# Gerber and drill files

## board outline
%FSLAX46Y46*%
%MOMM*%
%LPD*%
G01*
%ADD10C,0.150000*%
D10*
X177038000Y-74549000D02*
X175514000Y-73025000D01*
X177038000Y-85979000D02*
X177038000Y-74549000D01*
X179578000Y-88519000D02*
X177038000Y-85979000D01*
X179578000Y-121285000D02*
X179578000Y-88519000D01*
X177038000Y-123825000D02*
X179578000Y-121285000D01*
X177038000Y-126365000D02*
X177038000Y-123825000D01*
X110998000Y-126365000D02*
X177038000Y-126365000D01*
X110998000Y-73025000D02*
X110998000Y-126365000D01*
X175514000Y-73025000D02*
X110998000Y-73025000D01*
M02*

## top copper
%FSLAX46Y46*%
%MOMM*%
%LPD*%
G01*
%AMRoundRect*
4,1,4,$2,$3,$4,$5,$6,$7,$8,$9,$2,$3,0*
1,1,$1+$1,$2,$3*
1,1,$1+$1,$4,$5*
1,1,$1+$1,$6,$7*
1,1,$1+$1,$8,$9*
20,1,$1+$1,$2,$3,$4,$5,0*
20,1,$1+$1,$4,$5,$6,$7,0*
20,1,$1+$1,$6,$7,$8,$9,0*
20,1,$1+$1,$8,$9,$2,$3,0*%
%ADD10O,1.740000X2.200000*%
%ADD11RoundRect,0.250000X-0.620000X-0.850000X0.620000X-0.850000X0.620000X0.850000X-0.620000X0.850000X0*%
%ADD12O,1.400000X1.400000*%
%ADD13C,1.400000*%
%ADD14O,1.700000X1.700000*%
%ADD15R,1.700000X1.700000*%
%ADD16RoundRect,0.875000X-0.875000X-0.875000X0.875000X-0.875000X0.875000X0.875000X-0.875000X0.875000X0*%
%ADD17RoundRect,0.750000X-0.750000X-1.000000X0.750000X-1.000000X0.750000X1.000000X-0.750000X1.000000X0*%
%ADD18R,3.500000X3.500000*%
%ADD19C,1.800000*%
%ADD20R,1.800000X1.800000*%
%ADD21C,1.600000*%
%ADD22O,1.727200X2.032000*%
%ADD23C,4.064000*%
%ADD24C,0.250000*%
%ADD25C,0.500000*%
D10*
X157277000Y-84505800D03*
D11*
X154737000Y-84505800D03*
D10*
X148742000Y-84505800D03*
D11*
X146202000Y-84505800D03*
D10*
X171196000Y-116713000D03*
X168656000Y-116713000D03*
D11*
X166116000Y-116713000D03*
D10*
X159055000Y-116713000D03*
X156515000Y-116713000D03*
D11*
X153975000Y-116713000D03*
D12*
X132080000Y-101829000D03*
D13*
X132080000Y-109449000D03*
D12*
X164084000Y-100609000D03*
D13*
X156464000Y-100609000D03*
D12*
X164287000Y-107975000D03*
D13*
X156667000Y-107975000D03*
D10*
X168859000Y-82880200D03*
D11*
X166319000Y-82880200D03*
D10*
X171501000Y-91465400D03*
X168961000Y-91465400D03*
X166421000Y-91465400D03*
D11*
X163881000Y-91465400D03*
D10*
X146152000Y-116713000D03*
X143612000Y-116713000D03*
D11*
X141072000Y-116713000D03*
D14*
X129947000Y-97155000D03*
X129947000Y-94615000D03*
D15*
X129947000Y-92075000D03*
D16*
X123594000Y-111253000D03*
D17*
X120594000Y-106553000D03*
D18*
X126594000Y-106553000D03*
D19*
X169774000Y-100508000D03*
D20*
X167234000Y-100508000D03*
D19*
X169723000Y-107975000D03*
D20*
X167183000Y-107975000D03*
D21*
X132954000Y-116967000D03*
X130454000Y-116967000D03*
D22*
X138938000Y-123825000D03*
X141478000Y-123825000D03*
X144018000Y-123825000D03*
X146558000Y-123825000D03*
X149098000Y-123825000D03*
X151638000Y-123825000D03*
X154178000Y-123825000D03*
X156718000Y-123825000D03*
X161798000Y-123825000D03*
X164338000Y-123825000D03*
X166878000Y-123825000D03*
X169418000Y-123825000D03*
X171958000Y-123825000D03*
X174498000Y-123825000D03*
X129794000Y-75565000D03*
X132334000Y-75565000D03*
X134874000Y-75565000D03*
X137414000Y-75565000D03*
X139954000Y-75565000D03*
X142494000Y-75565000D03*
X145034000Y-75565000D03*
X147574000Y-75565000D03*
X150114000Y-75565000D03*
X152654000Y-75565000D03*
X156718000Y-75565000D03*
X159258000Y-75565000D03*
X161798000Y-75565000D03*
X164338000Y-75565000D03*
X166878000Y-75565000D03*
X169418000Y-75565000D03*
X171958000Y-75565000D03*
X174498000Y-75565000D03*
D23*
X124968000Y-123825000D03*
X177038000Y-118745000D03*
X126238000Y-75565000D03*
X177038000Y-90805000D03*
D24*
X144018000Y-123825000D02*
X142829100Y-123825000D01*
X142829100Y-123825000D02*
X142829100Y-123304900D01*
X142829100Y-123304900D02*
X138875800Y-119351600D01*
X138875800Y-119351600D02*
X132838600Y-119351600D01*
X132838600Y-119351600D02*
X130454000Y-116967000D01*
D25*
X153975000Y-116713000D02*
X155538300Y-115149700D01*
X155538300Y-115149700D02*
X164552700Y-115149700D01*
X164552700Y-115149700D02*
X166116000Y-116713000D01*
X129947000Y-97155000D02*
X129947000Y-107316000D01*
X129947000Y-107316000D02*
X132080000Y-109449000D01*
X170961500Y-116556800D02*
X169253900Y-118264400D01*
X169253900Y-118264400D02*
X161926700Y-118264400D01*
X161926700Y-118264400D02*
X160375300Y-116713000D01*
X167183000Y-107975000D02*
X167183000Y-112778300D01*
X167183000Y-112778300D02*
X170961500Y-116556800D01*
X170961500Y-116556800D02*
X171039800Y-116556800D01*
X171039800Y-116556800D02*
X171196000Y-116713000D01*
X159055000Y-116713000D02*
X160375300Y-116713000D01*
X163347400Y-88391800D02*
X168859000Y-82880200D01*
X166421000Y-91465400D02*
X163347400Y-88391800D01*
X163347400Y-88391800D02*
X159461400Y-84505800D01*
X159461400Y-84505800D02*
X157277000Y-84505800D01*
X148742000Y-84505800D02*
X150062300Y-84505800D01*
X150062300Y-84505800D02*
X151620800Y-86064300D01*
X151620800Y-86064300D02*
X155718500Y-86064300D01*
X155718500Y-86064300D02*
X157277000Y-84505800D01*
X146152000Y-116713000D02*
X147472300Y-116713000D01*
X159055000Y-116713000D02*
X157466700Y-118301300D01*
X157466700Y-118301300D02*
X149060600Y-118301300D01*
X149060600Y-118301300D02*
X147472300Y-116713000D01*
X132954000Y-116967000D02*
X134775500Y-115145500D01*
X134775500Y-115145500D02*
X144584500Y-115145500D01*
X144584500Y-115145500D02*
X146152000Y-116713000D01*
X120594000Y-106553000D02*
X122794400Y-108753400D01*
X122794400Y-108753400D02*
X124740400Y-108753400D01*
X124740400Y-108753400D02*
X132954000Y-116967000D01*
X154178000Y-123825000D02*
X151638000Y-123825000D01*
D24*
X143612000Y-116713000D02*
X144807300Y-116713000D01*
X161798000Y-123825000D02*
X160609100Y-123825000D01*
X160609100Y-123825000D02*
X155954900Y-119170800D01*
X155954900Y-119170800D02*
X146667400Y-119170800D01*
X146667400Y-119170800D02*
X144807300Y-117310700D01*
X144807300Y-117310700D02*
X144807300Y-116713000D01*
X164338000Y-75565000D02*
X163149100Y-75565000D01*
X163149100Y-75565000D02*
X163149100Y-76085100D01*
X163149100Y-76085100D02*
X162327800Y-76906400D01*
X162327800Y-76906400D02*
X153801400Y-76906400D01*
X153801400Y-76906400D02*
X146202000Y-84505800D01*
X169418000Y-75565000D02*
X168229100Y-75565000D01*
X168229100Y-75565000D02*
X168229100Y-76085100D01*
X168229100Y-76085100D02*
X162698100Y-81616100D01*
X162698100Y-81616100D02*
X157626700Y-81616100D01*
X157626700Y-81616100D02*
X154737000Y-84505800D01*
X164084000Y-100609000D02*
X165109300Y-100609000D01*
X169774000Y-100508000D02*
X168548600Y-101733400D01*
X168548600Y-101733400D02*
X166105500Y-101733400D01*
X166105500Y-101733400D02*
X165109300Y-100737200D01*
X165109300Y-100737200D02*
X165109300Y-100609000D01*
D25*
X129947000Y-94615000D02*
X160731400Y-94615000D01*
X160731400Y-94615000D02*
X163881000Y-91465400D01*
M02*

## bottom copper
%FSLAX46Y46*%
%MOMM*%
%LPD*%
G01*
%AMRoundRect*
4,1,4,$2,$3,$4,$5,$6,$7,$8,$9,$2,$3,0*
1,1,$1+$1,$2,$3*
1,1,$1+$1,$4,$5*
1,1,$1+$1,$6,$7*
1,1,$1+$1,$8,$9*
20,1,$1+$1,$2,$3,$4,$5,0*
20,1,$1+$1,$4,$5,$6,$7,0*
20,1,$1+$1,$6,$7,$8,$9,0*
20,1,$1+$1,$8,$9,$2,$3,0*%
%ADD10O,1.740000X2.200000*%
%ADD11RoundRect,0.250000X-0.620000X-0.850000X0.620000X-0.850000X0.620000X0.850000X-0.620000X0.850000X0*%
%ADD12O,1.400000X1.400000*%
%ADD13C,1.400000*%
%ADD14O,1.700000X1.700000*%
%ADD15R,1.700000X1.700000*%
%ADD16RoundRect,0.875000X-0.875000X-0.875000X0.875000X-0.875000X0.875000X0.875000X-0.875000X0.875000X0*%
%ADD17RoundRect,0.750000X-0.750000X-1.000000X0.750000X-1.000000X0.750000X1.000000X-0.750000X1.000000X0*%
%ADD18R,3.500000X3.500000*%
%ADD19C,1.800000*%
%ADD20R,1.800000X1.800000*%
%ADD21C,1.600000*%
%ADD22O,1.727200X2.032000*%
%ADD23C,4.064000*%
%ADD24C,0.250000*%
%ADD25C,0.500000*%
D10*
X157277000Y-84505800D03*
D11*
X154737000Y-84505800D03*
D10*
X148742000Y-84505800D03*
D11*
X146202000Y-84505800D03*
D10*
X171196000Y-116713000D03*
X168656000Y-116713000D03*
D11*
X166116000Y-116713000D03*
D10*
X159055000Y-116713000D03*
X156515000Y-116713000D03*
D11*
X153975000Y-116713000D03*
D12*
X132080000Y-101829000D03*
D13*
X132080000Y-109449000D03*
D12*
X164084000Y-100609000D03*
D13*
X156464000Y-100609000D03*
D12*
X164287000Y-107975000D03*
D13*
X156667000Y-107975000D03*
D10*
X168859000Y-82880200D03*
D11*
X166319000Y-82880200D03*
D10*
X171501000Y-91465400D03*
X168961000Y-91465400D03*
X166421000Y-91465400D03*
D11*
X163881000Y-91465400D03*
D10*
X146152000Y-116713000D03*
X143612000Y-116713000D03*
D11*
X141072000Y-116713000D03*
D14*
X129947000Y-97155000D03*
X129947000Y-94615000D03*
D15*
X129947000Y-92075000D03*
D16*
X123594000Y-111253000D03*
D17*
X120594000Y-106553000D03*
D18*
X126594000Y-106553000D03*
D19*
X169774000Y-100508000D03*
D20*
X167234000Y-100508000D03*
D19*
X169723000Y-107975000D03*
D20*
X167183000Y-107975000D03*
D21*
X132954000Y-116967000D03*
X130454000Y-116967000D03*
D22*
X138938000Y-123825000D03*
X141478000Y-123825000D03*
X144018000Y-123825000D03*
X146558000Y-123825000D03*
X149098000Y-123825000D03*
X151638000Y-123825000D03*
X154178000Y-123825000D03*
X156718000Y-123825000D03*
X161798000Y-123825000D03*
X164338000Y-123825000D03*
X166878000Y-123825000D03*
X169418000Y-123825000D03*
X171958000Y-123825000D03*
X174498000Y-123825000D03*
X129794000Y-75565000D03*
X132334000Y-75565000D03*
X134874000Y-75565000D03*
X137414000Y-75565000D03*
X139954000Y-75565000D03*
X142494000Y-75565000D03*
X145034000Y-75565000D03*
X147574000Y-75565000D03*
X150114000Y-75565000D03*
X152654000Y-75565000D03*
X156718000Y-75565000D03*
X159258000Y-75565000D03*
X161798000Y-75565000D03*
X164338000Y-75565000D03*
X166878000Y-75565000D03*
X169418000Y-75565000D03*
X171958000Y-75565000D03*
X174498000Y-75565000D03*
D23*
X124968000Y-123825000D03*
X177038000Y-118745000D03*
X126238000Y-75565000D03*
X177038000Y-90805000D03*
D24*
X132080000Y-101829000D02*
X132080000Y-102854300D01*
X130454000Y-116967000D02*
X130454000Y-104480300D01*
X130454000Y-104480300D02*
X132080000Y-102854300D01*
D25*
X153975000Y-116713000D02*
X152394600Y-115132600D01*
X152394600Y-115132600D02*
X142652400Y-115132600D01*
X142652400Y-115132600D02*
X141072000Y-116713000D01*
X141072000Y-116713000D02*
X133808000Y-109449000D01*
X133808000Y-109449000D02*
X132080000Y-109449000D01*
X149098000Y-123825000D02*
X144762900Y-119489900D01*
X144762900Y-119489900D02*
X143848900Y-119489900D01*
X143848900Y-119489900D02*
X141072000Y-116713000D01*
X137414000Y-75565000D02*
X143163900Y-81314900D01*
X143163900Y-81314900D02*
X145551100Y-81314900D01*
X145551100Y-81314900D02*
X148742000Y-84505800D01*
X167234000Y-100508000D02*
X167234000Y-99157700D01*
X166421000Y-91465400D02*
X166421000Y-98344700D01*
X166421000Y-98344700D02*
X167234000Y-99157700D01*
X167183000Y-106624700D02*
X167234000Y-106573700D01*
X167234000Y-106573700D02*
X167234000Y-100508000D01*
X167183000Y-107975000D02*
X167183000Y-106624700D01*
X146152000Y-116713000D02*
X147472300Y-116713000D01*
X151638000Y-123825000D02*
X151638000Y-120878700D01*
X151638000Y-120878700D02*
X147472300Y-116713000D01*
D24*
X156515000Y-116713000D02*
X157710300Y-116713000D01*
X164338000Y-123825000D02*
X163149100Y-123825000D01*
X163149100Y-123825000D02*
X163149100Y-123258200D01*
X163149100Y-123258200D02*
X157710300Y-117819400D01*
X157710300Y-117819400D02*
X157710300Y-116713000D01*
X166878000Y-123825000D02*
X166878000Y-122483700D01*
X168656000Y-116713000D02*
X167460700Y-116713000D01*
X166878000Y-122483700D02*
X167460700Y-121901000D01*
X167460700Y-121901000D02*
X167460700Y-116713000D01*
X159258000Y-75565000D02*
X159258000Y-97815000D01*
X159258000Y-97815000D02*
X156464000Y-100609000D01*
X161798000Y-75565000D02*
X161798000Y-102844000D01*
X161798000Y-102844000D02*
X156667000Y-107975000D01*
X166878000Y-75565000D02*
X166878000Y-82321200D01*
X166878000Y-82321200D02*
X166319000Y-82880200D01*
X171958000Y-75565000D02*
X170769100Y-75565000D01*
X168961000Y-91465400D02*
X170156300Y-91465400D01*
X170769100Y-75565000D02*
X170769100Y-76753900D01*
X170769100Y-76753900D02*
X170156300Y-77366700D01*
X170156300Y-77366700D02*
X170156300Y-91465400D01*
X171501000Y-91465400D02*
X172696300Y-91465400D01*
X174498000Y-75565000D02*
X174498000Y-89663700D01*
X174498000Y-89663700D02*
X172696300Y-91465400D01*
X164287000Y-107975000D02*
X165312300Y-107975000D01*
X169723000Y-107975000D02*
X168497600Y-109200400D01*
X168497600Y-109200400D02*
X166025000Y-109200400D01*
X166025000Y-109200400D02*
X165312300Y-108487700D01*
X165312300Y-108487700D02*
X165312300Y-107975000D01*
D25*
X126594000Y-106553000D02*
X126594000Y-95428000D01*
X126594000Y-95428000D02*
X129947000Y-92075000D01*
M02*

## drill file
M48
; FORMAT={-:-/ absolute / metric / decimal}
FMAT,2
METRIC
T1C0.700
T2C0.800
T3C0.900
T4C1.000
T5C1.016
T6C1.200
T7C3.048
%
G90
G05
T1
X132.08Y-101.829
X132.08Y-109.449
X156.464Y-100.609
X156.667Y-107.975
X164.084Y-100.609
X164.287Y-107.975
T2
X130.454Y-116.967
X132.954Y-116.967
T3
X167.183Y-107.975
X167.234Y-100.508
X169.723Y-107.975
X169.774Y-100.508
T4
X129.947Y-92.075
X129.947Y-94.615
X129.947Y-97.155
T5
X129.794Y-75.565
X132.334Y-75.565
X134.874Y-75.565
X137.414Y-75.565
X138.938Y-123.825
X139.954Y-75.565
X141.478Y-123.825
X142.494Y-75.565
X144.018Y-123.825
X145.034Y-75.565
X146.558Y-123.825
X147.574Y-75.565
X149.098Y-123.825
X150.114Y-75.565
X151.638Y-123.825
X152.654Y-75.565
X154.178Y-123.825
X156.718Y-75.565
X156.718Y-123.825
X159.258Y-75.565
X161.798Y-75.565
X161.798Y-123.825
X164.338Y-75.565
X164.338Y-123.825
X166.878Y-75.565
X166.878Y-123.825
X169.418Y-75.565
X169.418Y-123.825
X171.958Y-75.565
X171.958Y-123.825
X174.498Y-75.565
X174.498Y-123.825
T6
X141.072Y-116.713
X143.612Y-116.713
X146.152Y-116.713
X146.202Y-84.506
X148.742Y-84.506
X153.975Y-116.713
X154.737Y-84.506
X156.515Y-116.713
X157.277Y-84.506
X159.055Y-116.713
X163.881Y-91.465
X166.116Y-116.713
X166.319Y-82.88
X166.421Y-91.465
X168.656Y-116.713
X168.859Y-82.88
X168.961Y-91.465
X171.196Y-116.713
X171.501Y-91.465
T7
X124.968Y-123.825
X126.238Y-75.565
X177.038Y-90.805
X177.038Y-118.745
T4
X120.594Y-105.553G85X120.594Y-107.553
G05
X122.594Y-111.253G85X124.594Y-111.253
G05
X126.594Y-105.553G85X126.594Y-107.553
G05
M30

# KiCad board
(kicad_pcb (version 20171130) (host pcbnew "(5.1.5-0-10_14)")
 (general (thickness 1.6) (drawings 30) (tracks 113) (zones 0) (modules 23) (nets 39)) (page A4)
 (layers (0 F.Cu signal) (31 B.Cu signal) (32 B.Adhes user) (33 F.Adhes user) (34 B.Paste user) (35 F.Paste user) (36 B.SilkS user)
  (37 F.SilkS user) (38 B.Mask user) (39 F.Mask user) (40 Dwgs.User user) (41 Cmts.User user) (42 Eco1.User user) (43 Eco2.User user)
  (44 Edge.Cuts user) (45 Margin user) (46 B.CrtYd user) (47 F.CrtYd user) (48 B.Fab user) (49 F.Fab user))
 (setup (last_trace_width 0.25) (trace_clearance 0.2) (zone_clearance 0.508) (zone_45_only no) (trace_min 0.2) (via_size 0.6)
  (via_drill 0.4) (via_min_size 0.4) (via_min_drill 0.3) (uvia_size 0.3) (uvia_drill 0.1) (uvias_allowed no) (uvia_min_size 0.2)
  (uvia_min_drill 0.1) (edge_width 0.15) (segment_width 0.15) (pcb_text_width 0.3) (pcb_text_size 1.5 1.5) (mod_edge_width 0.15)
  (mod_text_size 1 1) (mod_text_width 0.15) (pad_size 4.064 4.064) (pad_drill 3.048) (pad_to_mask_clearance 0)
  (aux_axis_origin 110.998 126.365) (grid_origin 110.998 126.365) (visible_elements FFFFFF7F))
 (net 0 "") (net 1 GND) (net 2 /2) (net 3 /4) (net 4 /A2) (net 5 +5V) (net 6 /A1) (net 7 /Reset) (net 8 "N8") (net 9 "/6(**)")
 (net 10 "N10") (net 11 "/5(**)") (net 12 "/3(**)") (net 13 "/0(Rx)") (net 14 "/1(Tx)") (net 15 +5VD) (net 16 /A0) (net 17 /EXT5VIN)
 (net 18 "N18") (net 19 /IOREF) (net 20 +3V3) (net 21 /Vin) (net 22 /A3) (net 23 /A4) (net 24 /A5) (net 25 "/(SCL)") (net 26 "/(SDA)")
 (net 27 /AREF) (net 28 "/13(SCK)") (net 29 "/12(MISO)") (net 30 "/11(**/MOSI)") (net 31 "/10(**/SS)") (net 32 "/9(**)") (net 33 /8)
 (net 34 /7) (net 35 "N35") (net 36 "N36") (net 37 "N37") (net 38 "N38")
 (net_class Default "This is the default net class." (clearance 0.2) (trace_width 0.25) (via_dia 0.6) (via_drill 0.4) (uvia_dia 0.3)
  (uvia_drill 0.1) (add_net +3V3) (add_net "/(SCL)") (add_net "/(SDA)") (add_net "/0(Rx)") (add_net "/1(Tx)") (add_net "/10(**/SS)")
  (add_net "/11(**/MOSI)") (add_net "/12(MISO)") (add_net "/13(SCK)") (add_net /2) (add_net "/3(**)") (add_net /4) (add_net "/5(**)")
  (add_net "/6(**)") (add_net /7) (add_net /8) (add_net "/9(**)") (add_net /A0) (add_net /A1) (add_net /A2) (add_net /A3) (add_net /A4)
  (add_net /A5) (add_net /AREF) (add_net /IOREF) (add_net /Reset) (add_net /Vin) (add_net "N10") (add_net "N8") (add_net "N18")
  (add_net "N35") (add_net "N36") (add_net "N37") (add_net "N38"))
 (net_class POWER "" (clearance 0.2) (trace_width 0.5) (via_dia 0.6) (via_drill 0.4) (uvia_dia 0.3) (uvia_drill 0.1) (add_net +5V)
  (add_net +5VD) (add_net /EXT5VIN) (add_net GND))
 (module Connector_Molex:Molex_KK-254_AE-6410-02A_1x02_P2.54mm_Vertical (layer F.Cu) (at 154.737 84.5058)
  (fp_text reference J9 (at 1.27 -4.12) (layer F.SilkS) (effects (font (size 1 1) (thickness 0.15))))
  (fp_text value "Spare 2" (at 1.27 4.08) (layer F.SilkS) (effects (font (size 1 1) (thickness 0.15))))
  (pad 2 thru_hole oval (at 2.54 0) (size 1.74 2.2) (drill 1.2) (layers *.Cu *.Mask) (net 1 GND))
  (pad 1 thru_hole roundrect (at 0 0) (size 1.74 2.2) (drill 1.2) (layers *.Cu *.Mask) (roundrect_rratio 0.143678) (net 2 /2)))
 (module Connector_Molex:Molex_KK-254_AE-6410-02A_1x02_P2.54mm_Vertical (layer F.Cu) (at 146.202 84.5058)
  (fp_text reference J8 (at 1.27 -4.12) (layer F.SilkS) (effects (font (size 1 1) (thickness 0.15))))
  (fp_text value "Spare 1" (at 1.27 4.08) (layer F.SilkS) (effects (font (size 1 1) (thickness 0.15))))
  (pad 2 thru_hole oval (at 2.54 0) (size 1.74 2.2) (drill 1.2) (layers *.Cu *.Mask) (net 1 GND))
  (pad 1 thru_hole roundrect (at 0 0) (size 1.74 2.2) (drill 1.2) (layers *.Cu *.Mask) (roundrect_rratio 0.143678) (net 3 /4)))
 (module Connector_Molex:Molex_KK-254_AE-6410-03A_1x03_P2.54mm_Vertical (layer F.Cu) (at 166.116 116.713)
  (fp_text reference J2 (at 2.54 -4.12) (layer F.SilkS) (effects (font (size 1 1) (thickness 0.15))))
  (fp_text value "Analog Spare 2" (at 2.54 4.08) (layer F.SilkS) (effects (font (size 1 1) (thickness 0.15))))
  (pad 3 thru_hole oval (at 5.08 0) (size 1.74 2.2) (drill 1.2) (layers *.Cu *.Mask) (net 1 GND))
  (pad 2 thru_hole oval (at 2.54 0) (size 1.74 2.2) (drill 1.2) (layers *.Cu *.Mask) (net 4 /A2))
  (pad 1 thru_hole roundrect (at 0 0) (size 1.74 2.2) (drill 1.2) (layers *.Cu *.Mask) (roundrect_rratio 0.143678) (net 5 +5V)))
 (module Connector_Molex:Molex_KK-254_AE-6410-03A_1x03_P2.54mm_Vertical (layer F.Cu) (at 153.975 116.713)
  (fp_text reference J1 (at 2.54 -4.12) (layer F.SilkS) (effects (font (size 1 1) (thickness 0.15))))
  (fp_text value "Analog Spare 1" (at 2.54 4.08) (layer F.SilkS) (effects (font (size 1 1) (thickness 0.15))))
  (pad 3 thru_hole oval (at 5.08 0) (size 1.74 2.2) (drill 1.2) (layers *.Cu *.Mask) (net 1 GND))
  (pad 2 thru_hole oval (at 2.54 0) (size 1.74 2.2) (drill 1.2) (layers *.Cu *.Mask) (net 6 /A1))
  (pad 1 thru_hole roundrect (at 0 0) (size 1.74 2.2) (drill 1.2) (layers *.Cu *.Mask) (roundrect_rratio 0.143678) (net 5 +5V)))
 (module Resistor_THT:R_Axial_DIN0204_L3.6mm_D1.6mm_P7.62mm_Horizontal (layer F.Cu) (at 132.08 109.449 90)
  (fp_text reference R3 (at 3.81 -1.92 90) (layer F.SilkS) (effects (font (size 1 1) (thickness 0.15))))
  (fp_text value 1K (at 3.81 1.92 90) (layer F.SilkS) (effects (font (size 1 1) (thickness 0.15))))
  (pad 2 thru_hole oval (at 7.62 0 90) (size 1.4 1.4) (drill 0.7) (layers *.Cu *.Mask) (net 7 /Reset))
  (pad 1 thru_hole circle (at 0 0 90) (size 1.4 1.4) (drill 0.7) (layers *.Cu *.Mask) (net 5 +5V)))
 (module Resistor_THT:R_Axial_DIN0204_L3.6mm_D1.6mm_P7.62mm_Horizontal (layer F.Cu) (at 156.464 100.609)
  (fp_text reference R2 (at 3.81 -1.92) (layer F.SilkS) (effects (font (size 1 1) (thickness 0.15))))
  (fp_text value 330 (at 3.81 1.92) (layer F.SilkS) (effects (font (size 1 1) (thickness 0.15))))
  (pad 2 thru_hole oval (at 7.62 0) (size 1.4 1.4) (drill 0.7) (layers *.Cu *.Mask) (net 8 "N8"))
  (pad 1 thru_hole circle (at 0 0) (size 1.4 1.4) (drill 0.7) (layers *.Cu *.Mask) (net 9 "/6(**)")))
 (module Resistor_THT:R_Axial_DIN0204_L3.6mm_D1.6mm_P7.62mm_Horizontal (layer F.Cu) (at 156.667 107.975)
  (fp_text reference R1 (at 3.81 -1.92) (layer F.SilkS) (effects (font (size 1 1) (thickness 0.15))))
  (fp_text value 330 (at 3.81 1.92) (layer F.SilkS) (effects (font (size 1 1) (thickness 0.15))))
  (pad 2 thru_hole oval (at 7.62 0) (size 1.4 1.4) (drill 0.7) (layers *.Cu *.Mask) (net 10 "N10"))
  (pad 1 thru_hole circle (at 0 0) (size 1.4 1.4) (drill 0.7) (layers *.Cu *.Mask) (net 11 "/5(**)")))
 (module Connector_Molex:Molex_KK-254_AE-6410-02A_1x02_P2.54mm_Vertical (layer F.Cu) (at 166.319 82.8802)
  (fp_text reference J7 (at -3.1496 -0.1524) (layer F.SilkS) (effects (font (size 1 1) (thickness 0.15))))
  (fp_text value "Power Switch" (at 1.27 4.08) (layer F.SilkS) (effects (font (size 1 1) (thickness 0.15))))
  (pad 2 thru_hole oval (at 2.54 0) (size 1.74 2.2) (drill 1.2) (layers *.Cu *.Mask) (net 1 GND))
  (pad 1 thru_hole roundrect (at 0 0) (size 1.74 2.2) (drill 1.2) (layers *.Cu *.Mask) (roundrect_rratio 0.143678) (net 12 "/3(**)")))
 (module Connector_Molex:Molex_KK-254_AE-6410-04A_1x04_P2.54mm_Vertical (layer F.Cu) (at 163.881 91.4654)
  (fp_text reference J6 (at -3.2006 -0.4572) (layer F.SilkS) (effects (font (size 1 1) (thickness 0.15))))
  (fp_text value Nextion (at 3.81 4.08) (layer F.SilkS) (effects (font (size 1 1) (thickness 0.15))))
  (pad 4 thru_hole oval (at 7.62 0) (size 1.74 2.2) (drill 1.2) (layers *.Cu *.Mask) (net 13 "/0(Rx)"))
  (pad 3 thru_hole oval (at 5.08 0) (size 1.74 2.2) (drill 1.2) (layers *.Cu *.Mask) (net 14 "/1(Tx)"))
  (pad 2 thru_hole oval (at 2.54 0) (size 1.74 2.2) (drill 1.2) (layers *.Cu *.Mask) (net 1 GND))
  (pad 1 thru_hole roundrect (at 0 0) (size 1.74 2.2) (drill 1.2) (layers *.Cu *.Mask) (roundrect_rratio 0.143678) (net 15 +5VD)))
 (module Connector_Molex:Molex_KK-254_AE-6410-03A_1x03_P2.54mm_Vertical (layer F.Cu) (at 141.072 116.713)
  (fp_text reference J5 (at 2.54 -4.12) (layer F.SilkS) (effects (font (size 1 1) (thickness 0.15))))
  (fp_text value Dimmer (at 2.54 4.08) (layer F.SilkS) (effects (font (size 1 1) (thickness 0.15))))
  (pad 3 thru_hole oval (at 5.08 0) (size 1.74 2.2) (drill 1.2) (layers *.Cu *.Mask) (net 1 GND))
  (pad 2 thru_hole oval (at 2.54 0) (size 1.74 2.2) (drill 1.2) (layers *.Cu *.Mask) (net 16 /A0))
  (pad 1 thru_hole roundrect (at 0 0) (size 1.74 2.2) (drill 1.2) (layers *.Cu *.Mask) (roundrect_rratio 0.143678) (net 5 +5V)))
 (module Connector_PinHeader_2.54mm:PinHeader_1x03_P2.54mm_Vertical (layer F.Cu) (at 129.947 92.075)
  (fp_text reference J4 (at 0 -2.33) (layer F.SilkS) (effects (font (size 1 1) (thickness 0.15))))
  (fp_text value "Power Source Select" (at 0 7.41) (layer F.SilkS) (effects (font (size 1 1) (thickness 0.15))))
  (pad 3 thru_hole oval (at 0 5.08) (size 1.7 1.7) (drill 1) (layers *.Cu *.Mask) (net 5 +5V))
  (pad 2 thru_hole oval (at 0 2.54) (size 1.7 1.7) (drill 1) (layers *.Cu *.Mask) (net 15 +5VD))
  (pad 1 thru_hole rect (at 0 0) (size 1.7 1.7) (drill 1) (layers *.Cu *.Mask) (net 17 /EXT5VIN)))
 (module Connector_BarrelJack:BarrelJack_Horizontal (layer F.Cu) (at 126.594 106.553)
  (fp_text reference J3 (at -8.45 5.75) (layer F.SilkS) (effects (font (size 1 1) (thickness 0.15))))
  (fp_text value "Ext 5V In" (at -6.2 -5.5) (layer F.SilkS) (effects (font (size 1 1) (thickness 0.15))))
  (pad 3 thru_hole roundrect (at -3 4.7) (size 3.5 3.5) (drill oval 3 1) (layers *.Cu *.Mask) (roundrect_rratio 0.25))
  (pad 2 thru_hole roundrect (at -6 0) (size 3 3.5) (drill oval 1 3) (layers *.Cu *.Mask) (roundrect_rratio 0.25) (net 1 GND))
  (pad 1 thru_hole rect (at 0 0) (size 3.5 3.5) (drill oval 1 3) (layers *.Cu *.Mask) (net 17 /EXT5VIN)))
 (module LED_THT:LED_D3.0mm (layer F.Cu) (at 167.234 100.508)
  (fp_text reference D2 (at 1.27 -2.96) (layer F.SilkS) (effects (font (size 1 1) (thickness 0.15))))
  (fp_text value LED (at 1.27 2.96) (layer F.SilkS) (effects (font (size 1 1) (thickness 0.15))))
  (pad 2 thru_hole circle (at 2.54 0) (size 1.8 1.8) (drill 0.9) (layers *.Cu *.Mask) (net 8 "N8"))
  (pad 1 thru_hole rect (at 0 0) (size 1.8 1.8) (drill 0.9) (layers *.Cu *.Mask) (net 1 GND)))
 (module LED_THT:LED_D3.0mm (layer F.Cu) (at 167.183 107.975)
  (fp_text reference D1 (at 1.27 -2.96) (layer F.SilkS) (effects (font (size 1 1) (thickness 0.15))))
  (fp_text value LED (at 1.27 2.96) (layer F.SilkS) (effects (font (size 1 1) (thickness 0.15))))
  (pad 2 thru_hole circle (at 2.54 0) (size 1.8 1.8) (drill 0.9) (layers *.Cu *.Mask) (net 10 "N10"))
  (pad 1 thru_hole rect (at 0 0) (size 1.8 1.8) (drill 0.9) (layers *.Cu *.Mask) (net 1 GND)))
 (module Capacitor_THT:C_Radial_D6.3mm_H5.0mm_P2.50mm (layer F.Cu) (at 130.454 116.967)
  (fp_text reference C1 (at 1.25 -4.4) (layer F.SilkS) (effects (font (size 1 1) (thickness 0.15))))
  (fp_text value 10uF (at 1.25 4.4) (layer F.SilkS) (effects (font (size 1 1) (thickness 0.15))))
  (pad 2 thru_hole circle (at 2.5 0) (size 1.6 1.6) (drill 0.8) (layers *.Cu *.Mask) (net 1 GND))
  (pad 1 thru_hole circle (at 0 0) (size 1.6 1.6) (drill 0.8) (layers *.Cu *.Mask) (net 7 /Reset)))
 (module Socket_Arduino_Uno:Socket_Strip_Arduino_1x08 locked (layer F.Cu) (at 138.938 123.825)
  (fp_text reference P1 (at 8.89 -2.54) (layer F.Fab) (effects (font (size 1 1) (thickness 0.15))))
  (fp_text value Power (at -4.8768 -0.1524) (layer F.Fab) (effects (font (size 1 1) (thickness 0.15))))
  (pad 1 thru_hole oval (at 0 0) (size 1.7272 2.032) (drill 1.016) (layers *.Cu *.Mask F.SilkS) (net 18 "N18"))
  (pad 2 thru_hole oval (at 2.54 0) (size 1.7272 2.032) (drill 1.016) (layers *.Cu *.Mask F.SilkS) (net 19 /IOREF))
  (pad 3 thru_hole oval (at 5.08 0) (size 1.7272 2.032) (drill 1.016) (layers *.Cu *.Mask F.SilkS) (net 7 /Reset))
  (pad 4 thru_hole oval (at 7.62 0) (size 1.7272 2.032) (drill 1.016) (layers *.Cu *.Mask F.SilkS) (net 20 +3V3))
  (pad 5 thru_hole oval (at 10.16 0) (size 1.7272 2.032) (drill 1.016) (layers *.Cu *.Mask F.SilkS) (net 5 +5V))
  (pad 6 thru_hole oval (at 12.7 0) (size 1.7272 2.032) (drill 1.016) (layers *.Cu *.Mask F.SilkS) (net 1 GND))
  (pad 7 thru_hole oval (at 15.24 0) (size 1.7272 2.032) (drill 1.016) (layers *.Cu *.Mask F.SilkS) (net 1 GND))
  (pad 8 thru_hole oval (at 17.78 0) (size 1.7272 2.032) (drill 1.016) (layers *.Cu *.Mask F.SilkS) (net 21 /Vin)))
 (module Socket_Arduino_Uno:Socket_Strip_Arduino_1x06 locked (layer F.Cu) (at 161.798 123.825)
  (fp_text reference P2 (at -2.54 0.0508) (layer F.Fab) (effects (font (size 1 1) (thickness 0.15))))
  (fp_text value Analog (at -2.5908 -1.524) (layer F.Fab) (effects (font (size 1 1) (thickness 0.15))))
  (pad 1 thru_hole oval (at 0 0) (size 1.7272 2.032) (drill 1.016) (layers *.Cu *.Mask F.SilkS) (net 16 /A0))
  (pad 2 thru_hole oval (at 2.54 0) (size 1.7272 2.032) (drill 1.016) (layers *.Cu *.Mask F.SilkS) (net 6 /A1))
  (pad 3 thru_hole oval (at 5.08 0) (size 1.7272 2.032) (drill 1.016) (layers *.Cu *.Mask F.SilkS) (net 4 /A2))
  (pad 4 thru_hole oval (at 7.62 0) (size 1.7272 2.032) (drill 1.016) (layers *.Cu *.Mask F.SilkS) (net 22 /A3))
  (pad 5 thru_hole oval (at 10.16 0) (size 1.7272 2.032) (drill 1.016) (layers *.Cu *.Mask F.SilkS) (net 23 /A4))
  (pad 6 thru_hole oval (at 12.7 0) (size 1.7272 2.032) (drill 1.016) (layers *.Cu *.Mask F.SilkS) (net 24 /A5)))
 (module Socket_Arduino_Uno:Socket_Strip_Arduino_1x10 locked (layer F.Cu) (at 129.794 75.565)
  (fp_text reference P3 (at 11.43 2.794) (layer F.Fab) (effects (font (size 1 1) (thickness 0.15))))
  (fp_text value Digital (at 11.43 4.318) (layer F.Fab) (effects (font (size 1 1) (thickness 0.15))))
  (pad 1 thru_hole oval (at 0 0) (size 1.7272 2.032) (drill 1.016) (layers *.Cu *.Mask F.SilkS) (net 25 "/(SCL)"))
  (pad 2 thru_hole oval (at 2.54 0) (size 1.7272 2.032) (drill 1.016) (layers *.Cu *.Mask F.SilkS) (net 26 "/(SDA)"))
  (pad 3 thru_hole oval (at 5.08 0) (size 1.7272 2.032) (drill 1.016) (layers *.Cu *.Mask F.SilkS) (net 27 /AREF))
  (pad 4 thru_hole oval (at 7.62 0) (size 1.7272 2.032) (drill 1.016) (layers *.Cu *.Mask F.SilkS) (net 1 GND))
  (pad 5 thru_hole oval (at 10.16 0) (size 1.7272 2.032) (drill 1.016) (layers *.Cu *.Mask F.SilkS) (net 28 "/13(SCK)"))
  (pad 6 thru_hole oval (at 12.7 0) (size 1.7272 2.032) (drill 1.016) (layers *.Cu *.Mask F.SilkS) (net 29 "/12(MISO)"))
  (pad 7 thru_hole oval (at 15.24 0) (size 1.7272 2.032) (drill 1.016) (layers *.Cu *.Mask F.SilkS) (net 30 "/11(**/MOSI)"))
  (pad 8 thru_hole oval (at 17.78 0) (size 1.7272 2.032) (drill 1.016) (layers *.Cu *.Mask F.SilkS) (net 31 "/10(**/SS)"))
  (pad 9 thru_hole oval (at 20.32 0) (size 1.7272 2.032) (drill 1.016) (layers *.Cu *.Mask F.SilkS) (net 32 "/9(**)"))
  (pad 10 thru_hole oval (at 22.86 0) (size 1.7272 2.032) (drill 1.016) (layers *.Cu *.Mask F.SilkS) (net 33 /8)))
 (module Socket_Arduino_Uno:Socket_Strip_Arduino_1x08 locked (layer F.Cu) (at 156.718 75.565)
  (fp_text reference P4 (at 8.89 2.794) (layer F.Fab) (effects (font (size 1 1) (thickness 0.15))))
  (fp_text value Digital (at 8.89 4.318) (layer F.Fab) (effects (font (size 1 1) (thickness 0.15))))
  (pad 1 thru_hole oval (at 0 0) (size 1.7272 2.032) (drill 1.016) (layers *.Cu *.Mask F.SilkS) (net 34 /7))
  (pad 2 thru_hole oval (at 2.54 0) (size 1.7272 2.032) (drill 1.016) (layers *.Cu *.Mask F.SilkS) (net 9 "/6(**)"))
  (pad 3 thru_hole oval (at 5.08 0) (size 1.7272 2.032) (drill 1.016) (layers *.Cu *.Mask F.SilkS) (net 11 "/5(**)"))
  (pad 4 thru_hole oval (at 7.62 0) (size 1.7272 2.032) (drill 1.016) (layers *.Cu *.Mask F.SilkS) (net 3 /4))
  (pad 5 thru_hole oval (at 10.16 0) (size 1.7272 2.032) (drill 1.016) (layers *.Cu *.Mask F.SilkS) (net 12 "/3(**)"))
  (pad 6 thru_hole oval (at 12.7 0) (size 1.7272 2.032) (drill 1.016) (layers *.Cu *.Mask F.SilkS) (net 2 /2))
  (pad 7 thru_hole oval (at 15.24 0) (size 1.7272 2.032) (drill 1.016) (layers *.Cu *.Mask F.SilkS) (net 14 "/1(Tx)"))
  (pad 8 thru_hole oval (at 17.78 0) (size 1.7272 2.032) (drill 1.016) (layers *.Cu *.Mask F.SilkS) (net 13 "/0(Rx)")))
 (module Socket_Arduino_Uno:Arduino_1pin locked (layer F.Cu) (at 124.968 123.825)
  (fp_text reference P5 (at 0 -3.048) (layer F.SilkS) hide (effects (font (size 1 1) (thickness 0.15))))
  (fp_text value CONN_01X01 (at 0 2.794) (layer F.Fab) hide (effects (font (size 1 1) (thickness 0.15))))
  (pad 1 thru_hole circle (at 0 0) (size 4.064 4.064) (drill 3.048) (layers *.Cu *.Mask F.SilkS) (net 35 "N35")))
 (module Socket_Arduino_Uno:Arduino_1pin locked (layer F.Cu) (at 177.038 118.745)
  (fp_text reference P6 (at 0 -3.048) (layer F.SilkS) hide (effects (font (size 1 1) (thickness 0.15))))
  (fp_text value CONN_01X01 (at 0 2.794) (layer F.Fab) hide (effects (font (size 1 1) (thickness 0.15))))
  (pad 1 thru_hole circle (at 0 0) (size 4.064 4.064) (drill 3.048) (layers *.Cu *.Mask F.SilkS) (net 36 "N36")))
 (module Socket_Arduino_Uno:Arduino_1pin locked (layer F.Cu) (at 126.238 75.565)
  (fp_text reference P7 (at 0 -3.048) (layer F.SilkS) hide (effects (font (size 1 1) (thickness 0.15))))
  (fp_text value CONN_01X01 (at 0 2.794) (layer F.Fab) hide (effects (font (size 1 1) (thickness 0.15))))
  (pad 1 thru_hole circle (at 0 0) (size 4.064 4.064) (drill 3.048) (layers *.Cu *.Mask F.SilkS) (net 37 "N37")))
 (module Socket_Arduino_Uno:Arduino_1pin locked (layer F.Cu) (at 177.038 90.805)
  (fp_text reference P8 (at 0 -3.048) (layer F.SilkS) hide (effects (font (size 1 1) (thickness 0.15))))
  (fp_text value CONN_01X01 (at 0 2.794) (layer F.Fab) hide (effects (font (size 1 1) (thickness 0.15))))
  (pad 1 thru_hole circle (at 0 0) (size 4.064 4.064) (drill 3.048) (layers *.Cu *.Mask F.SilkS) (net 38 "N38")))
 (gr_line (start 177.038 74.549) (end 175.514 73.025) (angle 90) (layer Edge.Cuts) (width 0.15))
 (gr_line (start 177.038 85.979) (end 177.038 74.549) (angle 90) (layer Edge.Cuts) (width 0.15))
 (gr_line (start 179.578 88.519) (end 177.038 85.979) (angle 90) (layer Edge.Cuts) (width 0.15))
 (gr_line (start 179.578 121.285) (end 179.578 88.519) (angle 90) (layer Edge.Cuts) (width 0.15))
 (gr_line (start 177.038 123.825) (end 179.578 121.285) (angle 90) (layer Edge.Cuts) (width 0.15))
 (gr_line (start 177.038 126.365) (end 177.038 123.825) (angle 90) (layer Edge.Cuts) (width 0.15))
 (gr_line (start 110.998 126.365) (end 177.038 126.365) (angle 90) (layer Edge.Cuts) (width 0.15))
 (gr_line (start 110.998 73.025) (end 110.998 126.365) (angle 90) (layer Edge.Cuts) (width 0.15))
 (gr_line (start 175.514 73.025) (end 110.998 73.025) (angle 90) (layer Edge.Cuts) (width 0.15))
 (segment (start 132.08 101.829) (end 132.08 102.8543) (width 0.25) (layer B.Cu) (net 7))
 (segment (start 130.454 116.967) (end 130.454 104.4803) (width 0.25) (layer B.Cu) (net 7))
 (segment (start 130.454 104.4803) (end 132.08 102.8543) (width 0.25) (layer B.Cu) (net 7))
 (segment (start 144.018 123.825) (end 142.8291 123.825) (width 0.25) (layer F.Cu) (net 7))
 (segment (start 142.8291 123.825) (end 142.8291 123.3049) (width 0.25) (layer F.Cu) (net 7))
 (segment (start 142.8291 123.3049) (end 138.8758 119.3516) (width 0.25) (layer F.Cu) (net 7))
 (segment (start 138.8758 119.3516) (end 132.8386 119.3516) (width 0.25) (layer F.Cu) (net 7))
 (segment (start 132.8386 119.3516) (end 130.454 116.967) (width 0.25) (layer F.Cu) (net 7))
 (segment (start 153.975 116.713) (end 155.5383 115.1497) (width 0.5) (layer F.Cu) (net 5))
 (segment (start 155.5383 115.1497) (end 164.5527 115.1497) (width 0.5) (layer F.Cu) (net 5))
 (segment (start 164.5527 115.1497) (end 166.116 116.713) (width 0.5) (layer F.Cu) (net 5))
 (segment (start 153.975 116.713) (end 152.3946 115.1326) (width 0.5) (layer B.Cu) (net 5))
 (segment (start 152.3946 115.1326) (end 142.6524 115.1326) (width 0.5) (layer B.Cu) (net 5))
 (segment (start 142.6524 115.1326) (end 141.072 116.713) (width 0.5) (layer B.Cu) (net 5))
 (segment (start 141.072 116.713) (end 133.808 109.449) (width 0.5) (layer B.Cu) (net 5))
 (segment (start 133.808 109.449) (end 132.08 109.449) (width 0.5) (layer B.Cu) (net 5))
 (segment (start 129.947 97.155) (end 129.947 107.316) (width 0.5) (layer F.Cu) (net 5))
 (segment (start 129.947 107.316) (end 132.08 109.449) (width 0.5) (layer F.Cu) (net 5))
 (segment (start 149.098 123.825) (end 144.7629 119.4899) (width 0.5) (layer B.Cu) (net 5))
 (segment (start 144.7629 119.4899) (end 143.8489 119.4899) (width 0.5) (layer B.Cu) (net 5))
 (segment (start 143.8489 119.4899) (end 141.072 116.713) (width 0.5) (layer B.Cu) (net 5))
 (segment (start 137.414 75.565) (end 143.1639 81.3149) (width 0.5) (layer B.Cu) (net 1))
 (segment (start 143.1639 81.3149) (end 145.5511 81.3149) (width 0.5) (layer B.Cu) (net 1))
 (segment (start 145.5511 81.3149) (end 148.742 84.5058) (width 0.5) (layer B.Cu) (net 1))
 (segment (start 170.9615 116.5568) (end 169.2539 118.2644) (width 0.5) (layer F.Cu) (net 1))
 (segment (start 169.2539 118.2644) (end 161.9267 118.2644) (width 0.5) (layer F.Cu) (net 1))
 (segment (start 161.9267 118.2644) (end 160.3753 116.713) (width 0.5) (layer F.Cu) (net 1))
 (segment (start 167.183 107.975) (end 167.183 112.7783) (width 0.5) (layer F.Cu) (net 1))
 (segment (start 167.183 112.7783) (end 170.9615 116.5568) (width 0.5) (layer F.Cu) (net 1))
 (segment (start 170.9615 116.5568) (end 171.0398 116.5568) (width 0.5) (layer F.Cu) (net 1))
 (segment (start 171.0398 116.5568) (end 171.196 116.713) (width 0.5) (layer F.Cu) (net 1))
 (segment (start 159.055 116.713) (end 160.3753 116.713) (width 0.5) (layer F.Cu) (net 1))
 (segment (start 167.234 100.508) (end 167.234 99.1577) (width 0.5) (layer B.Cu) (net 1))
 (segment (start 166.421 91.4654) (end 166.421 98.3447) (width 0.5) (layer B.Cu) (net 1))
 (segment (start 166.421 98.3447) (end 167.234 99.1577) (width 0.5) (layer B.Cu) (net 1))
 (segment (start 163.3474 88.3918) (end 168.859 82.8802) (width 0.5) (layer F.Cu) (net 1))
 (segment (start 166.421 91.4654) (end 163.3474 88.3918) (width 0.5) (layer F.Cu) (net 1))
 (segment (start 163.3474 88.3918) (end 159.4614 84.5058) (width 0.5) (layer F.Cu) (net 1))
 (segment (start 159.4614 84.5058) (end 157.277 84.5058) (width 0.5) (layer F.Cu) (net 1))
 (segment (start 148.742 84.5058) (end 150.0623 84.5058) (width 0.5) (layer F.Cu) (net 1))
 (segment (start 150.0623 84.5058) (end 151.6208 86.0643) (width 0.5) (layer F.Cu) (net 1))
 (segment (start 151.6208 86.0643) (end 155.7185 86.0643) (width 0.5) (layer F.Cu) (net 1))
 (segment (start 155.7185 86.0643) (end 157.277 84.5058) (width 0.5) (layer F.Cu) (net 1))
 (segment (start 146.152 116.713) (end 147.4723 116.713) (width 0.5) (layer F.Cu) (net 1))
 (segment (start 159.055 116.713) (end 157.4667 118.3013) (width 0.5) (layer F.Cu) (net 1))
 (segment (start 157.4667 118.3013) (end 149.0606 118.3013) (width 0.5) (layer F.Cu) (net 1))
 (segment (start 149.0606 118.3013) (end 147.4723 116.713) (width 0.5) (layer F.Cu) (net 1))
 (segment (start 132.954 116.967) (end 134.7755 115.1455) (width 0.5) (layer F.Cu) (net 1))
 (segment (start 134.7755 115.1455) (end 144.5845 115.1455) (width 0.5) (layer F.Cu) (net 1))
 (segment (start 144.5845 115.1455) (end 146.152 116.713) (width 0.5) (layer F.Cu) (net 1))
 (segment (start 167.183 106.6247) (end 167.234 106.5737) (width 0.5) (layer B.Cu) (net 1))
 (segment (start 167.234 106.5737) (end 167.234 100.508) (width 0.5) (layer B.Cu) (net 1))
 (segment (start 120.594 106.553) (end 122.7944 108.7534) (width 0.5) (layer F.Cu) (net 1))
 (segment (start 122.7944 108.7534) (end 124.7404 108.7534) (width 0.5) (layer F.Cu) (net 1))
 (segment (start 124.7404 108.7534) (end 132.954 116.967) (width 0.5) (layer F.Cu) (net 1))
 (segment (start 167.183 107.975) (end 167.183 106.6247) (width 0.5) (layer B.Cu) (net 1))
 (segment (start 146.152 116.713) (end 147.4723 116.713) (width 0.5) (layer B.Cu) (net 1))
 (segment (start 151.638 123.825) (end 151.638 120.8787) (width 0.5) (layer B.Cu) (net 1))
 (segment (start 151.638 120.8787) (end 147.4723 116.713) (width 0.5) (layer B.Cu) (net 1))
 (segment (start 154.178 123.825) (end 151.638 123.825) (width 0.5) (layer F.Cu) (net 1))
 (segment (start 143.612 116.713) (end 144.8073 116.713) (width 0.25) (layer F.Cu) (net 16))
 (segment (start 161.798 123.825) (end 160.6091 123.825) (width 0.25) (layer F.Cu) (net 16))
 (segment (start 160.6091 123.825) (end 155.9549 119.1708) (width 0.25) (layer F.Cu) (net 16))
 (segment (start 155.9549 119.1708) (end 146.6674 119.1708) (width 0.25) (layer F.Cu) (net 16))
 (segment (start 146.6674 119.1708) (end 144.8073 117.3107) (width 0.25) (layer F.Cu) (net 16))
 (segment (start 144.8073 117.3107) (end 144.8073 116.713) (width 0.25) (layer F.Cu) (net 16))
 (segment (start 156.515 116.713) (end 157.7103 116.713) (width 0.25) (layer B.Cu) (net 6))
 (segment (start 164.338 123.825) (end 163.1491 123.825) (width 0.25) (layer B.Cu) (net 6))
 (segment (start 163.1491 123.825) (end 163.1491 123.2582) (width 0.25) (layer B.Cu) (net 6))
 (segment (start 163.1491 123.2582) (end 157.7103 117.8194) (width 0.25) (layer B.Cu) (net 6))
 (segment (start 157.7103 117.8194) (end 157.7103 116.713) (width 0.25) (layer B.Cu) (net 6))
 (segment (start 166.878 123.825) (end 166.878 122.4837) (width 0.25) (layer B.Cu) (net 4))
 (segment (start 168.656 116.713) (end 167.4607 116.713) (width 0.25) (layer B.Cu) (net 4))
 (segment (start 166.878 122.4837) (end 167.4607 121.901) (width 0.25) (layer B.Cu) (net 4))
 (segment (start 167.4607 121.901) (end 167.4607 116.713) (width 0.25) (layer B.Cu) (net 4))
 (segment (start 159.258 75.565) (end 159.258 97.815) (width 0.25) (layer B.Cu) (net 9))
 (segment (start 159.258 97.815) (end 156.464 100.609) (width 0.25) (layer B.Cu) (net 9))
 (segment (start 161.798 75.565) (end 161.798 102.844) (width 0.25) (layer B.Cu) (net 11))
 (segment (start 161.798 102.844) (end 156.667 107.975) (width 0.25) (layer B.Cu) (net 11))
 (segment (start 164.338 75.565) (end 163.1491 75.565) (width 0.25) (layer F.Cu) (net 3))
 (segment (start 163.1491 75.565) (end 163.1491 76.0851) (width 0.25) (layer F.Cu) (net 3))
 (segment (start 163.1491 76.0851) (end 162.3278 76.9064) (width 0.25) (layer F.Cu) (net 3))
 (segment (start 162.3278 76.9064) (end 153.8014 76.9064) (width 0.25) (layer F.Cu) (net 3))
 (segment (start 153.8014 76.9064) (end 146.202 84.5058) (width 0.25) (layer F.Cu) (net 3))
 (segment (start 166.878 75.565) (end 166.878 82.3212) (width 0.25) (layer B.Cu) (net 12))
 (segment (start 166.878 82.3212) (end 166.319 82.8802) (width 0.25) (layer B.Cu) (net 12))
 (segment (start 169.418 75.565) (end 168.2291 75.565) (width 0.25) (layer F.Cu) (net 2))
 (segment (start 168.2291 75.565) (end 168.2291 76.0851) (width 0.25) (layer F.Cu) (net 2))
 (segment (start 168.2291 76.0851) (end 162.6981 81.6161) (width 0.25) (layer F.Cu) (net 2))
 (segment (start 162.6981 81.6161) (end 157.6267 81.6161) (width 0.25) (layer F.Cu) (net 2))
 (segment (start 157.6267 81.6161) (end 154.737 84.5058) (width 0.25) (layer F.Cu) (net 2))
 (segment (start 171.958 75.565) (end 170.7691 75.565) (width 0.25) (layer B.Cu) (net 14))
 (segment (start 168.961 91.4654) (end 170.1563 91.4654) (width 0.25) (layer B.Cu) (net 14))
 (segment (start 170.7691 75.565) (end 170.7691 76.7539) (width 0.25) (layer B.Cu) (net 14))
 (segment (start 170.7691 76.7539) (end 170.1563 77.3667) (width 0.25) (layer B.Cu) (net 14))
 (segment (start 170.1563 77.3667) (end 170.1563 91.4654) (width 0.25) (layer B.Cu) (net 14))
 (segment (start 171.501 91.4654) (end 172.6963 91.4654) (width 0.25) (layer B.Cu) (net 13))
 (segment (start 174.498 75.565) (end 174.498 89.6637) (width 0.25) (layer B.Cu) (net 13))
 (segment (start 174.498 89.6637) (end 172.6963 91.4654) (width 0.25) (layer B.Cu) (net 13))
 (segment (start 164.287 107.975) (end 165.3123 107.975) (width 0.25) (layer B.Cu) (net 10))
 (segment (start 169.723 107.975) (end 168.4976 109.2004) (width 0.25) (layer B.Cu) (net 10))
 (segment (start 168.4976 109.2004) (end 166.025 109.2004) (width 0.25) (layer B.Cu) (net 10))
 (segment (start 166.025 109.2004) (end 165.3123 108.4877) (width 0.25) (layer B.Cu) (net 10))
 (segment (start 165.3123 108.4877) (end 165.3123 107.975) (width 0.25) (layer B.Cu) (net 10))
 (segment (start 164.084 100.609) (end 165.1093 100.609) (width 0.25) (layer F.Cu) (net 8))
 (segment (start 169.774 100.508) (end 168.5486 101.7334) (width 0.25) (layer F.Cu) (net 8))
 (segment (start 168.5486 101.7334) (end 166.1055 101.7334) (width 0.25) (layer F.Cu) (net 8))
 (segment (start 166.1055 101.7334) (end 165.1093 100.7372) (width 0.25) (layer F.Cu) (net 8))
 (segment (start 165.1093 100.7372) (end 165.1093 100.609) (width 0.25) (layer F.Cu) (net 8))
 (segment (start 129.947 94.615) (end 160.7314 94.615) (width 0.5) (layer F.Cu) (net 15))
 (segment (start 160.7314 94.615) (end 163.881 91.4654) (width 0.5) (layer F.Cu) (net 15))
 (segment (start 126.594 106.553) (end 126.594 95.428) (width 0.5) (layer B.Cu) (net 17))
 (segment (start 126.594 95.428) (end 129.947 92.075) (width 0.5) (layer B.Cu) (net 17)))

